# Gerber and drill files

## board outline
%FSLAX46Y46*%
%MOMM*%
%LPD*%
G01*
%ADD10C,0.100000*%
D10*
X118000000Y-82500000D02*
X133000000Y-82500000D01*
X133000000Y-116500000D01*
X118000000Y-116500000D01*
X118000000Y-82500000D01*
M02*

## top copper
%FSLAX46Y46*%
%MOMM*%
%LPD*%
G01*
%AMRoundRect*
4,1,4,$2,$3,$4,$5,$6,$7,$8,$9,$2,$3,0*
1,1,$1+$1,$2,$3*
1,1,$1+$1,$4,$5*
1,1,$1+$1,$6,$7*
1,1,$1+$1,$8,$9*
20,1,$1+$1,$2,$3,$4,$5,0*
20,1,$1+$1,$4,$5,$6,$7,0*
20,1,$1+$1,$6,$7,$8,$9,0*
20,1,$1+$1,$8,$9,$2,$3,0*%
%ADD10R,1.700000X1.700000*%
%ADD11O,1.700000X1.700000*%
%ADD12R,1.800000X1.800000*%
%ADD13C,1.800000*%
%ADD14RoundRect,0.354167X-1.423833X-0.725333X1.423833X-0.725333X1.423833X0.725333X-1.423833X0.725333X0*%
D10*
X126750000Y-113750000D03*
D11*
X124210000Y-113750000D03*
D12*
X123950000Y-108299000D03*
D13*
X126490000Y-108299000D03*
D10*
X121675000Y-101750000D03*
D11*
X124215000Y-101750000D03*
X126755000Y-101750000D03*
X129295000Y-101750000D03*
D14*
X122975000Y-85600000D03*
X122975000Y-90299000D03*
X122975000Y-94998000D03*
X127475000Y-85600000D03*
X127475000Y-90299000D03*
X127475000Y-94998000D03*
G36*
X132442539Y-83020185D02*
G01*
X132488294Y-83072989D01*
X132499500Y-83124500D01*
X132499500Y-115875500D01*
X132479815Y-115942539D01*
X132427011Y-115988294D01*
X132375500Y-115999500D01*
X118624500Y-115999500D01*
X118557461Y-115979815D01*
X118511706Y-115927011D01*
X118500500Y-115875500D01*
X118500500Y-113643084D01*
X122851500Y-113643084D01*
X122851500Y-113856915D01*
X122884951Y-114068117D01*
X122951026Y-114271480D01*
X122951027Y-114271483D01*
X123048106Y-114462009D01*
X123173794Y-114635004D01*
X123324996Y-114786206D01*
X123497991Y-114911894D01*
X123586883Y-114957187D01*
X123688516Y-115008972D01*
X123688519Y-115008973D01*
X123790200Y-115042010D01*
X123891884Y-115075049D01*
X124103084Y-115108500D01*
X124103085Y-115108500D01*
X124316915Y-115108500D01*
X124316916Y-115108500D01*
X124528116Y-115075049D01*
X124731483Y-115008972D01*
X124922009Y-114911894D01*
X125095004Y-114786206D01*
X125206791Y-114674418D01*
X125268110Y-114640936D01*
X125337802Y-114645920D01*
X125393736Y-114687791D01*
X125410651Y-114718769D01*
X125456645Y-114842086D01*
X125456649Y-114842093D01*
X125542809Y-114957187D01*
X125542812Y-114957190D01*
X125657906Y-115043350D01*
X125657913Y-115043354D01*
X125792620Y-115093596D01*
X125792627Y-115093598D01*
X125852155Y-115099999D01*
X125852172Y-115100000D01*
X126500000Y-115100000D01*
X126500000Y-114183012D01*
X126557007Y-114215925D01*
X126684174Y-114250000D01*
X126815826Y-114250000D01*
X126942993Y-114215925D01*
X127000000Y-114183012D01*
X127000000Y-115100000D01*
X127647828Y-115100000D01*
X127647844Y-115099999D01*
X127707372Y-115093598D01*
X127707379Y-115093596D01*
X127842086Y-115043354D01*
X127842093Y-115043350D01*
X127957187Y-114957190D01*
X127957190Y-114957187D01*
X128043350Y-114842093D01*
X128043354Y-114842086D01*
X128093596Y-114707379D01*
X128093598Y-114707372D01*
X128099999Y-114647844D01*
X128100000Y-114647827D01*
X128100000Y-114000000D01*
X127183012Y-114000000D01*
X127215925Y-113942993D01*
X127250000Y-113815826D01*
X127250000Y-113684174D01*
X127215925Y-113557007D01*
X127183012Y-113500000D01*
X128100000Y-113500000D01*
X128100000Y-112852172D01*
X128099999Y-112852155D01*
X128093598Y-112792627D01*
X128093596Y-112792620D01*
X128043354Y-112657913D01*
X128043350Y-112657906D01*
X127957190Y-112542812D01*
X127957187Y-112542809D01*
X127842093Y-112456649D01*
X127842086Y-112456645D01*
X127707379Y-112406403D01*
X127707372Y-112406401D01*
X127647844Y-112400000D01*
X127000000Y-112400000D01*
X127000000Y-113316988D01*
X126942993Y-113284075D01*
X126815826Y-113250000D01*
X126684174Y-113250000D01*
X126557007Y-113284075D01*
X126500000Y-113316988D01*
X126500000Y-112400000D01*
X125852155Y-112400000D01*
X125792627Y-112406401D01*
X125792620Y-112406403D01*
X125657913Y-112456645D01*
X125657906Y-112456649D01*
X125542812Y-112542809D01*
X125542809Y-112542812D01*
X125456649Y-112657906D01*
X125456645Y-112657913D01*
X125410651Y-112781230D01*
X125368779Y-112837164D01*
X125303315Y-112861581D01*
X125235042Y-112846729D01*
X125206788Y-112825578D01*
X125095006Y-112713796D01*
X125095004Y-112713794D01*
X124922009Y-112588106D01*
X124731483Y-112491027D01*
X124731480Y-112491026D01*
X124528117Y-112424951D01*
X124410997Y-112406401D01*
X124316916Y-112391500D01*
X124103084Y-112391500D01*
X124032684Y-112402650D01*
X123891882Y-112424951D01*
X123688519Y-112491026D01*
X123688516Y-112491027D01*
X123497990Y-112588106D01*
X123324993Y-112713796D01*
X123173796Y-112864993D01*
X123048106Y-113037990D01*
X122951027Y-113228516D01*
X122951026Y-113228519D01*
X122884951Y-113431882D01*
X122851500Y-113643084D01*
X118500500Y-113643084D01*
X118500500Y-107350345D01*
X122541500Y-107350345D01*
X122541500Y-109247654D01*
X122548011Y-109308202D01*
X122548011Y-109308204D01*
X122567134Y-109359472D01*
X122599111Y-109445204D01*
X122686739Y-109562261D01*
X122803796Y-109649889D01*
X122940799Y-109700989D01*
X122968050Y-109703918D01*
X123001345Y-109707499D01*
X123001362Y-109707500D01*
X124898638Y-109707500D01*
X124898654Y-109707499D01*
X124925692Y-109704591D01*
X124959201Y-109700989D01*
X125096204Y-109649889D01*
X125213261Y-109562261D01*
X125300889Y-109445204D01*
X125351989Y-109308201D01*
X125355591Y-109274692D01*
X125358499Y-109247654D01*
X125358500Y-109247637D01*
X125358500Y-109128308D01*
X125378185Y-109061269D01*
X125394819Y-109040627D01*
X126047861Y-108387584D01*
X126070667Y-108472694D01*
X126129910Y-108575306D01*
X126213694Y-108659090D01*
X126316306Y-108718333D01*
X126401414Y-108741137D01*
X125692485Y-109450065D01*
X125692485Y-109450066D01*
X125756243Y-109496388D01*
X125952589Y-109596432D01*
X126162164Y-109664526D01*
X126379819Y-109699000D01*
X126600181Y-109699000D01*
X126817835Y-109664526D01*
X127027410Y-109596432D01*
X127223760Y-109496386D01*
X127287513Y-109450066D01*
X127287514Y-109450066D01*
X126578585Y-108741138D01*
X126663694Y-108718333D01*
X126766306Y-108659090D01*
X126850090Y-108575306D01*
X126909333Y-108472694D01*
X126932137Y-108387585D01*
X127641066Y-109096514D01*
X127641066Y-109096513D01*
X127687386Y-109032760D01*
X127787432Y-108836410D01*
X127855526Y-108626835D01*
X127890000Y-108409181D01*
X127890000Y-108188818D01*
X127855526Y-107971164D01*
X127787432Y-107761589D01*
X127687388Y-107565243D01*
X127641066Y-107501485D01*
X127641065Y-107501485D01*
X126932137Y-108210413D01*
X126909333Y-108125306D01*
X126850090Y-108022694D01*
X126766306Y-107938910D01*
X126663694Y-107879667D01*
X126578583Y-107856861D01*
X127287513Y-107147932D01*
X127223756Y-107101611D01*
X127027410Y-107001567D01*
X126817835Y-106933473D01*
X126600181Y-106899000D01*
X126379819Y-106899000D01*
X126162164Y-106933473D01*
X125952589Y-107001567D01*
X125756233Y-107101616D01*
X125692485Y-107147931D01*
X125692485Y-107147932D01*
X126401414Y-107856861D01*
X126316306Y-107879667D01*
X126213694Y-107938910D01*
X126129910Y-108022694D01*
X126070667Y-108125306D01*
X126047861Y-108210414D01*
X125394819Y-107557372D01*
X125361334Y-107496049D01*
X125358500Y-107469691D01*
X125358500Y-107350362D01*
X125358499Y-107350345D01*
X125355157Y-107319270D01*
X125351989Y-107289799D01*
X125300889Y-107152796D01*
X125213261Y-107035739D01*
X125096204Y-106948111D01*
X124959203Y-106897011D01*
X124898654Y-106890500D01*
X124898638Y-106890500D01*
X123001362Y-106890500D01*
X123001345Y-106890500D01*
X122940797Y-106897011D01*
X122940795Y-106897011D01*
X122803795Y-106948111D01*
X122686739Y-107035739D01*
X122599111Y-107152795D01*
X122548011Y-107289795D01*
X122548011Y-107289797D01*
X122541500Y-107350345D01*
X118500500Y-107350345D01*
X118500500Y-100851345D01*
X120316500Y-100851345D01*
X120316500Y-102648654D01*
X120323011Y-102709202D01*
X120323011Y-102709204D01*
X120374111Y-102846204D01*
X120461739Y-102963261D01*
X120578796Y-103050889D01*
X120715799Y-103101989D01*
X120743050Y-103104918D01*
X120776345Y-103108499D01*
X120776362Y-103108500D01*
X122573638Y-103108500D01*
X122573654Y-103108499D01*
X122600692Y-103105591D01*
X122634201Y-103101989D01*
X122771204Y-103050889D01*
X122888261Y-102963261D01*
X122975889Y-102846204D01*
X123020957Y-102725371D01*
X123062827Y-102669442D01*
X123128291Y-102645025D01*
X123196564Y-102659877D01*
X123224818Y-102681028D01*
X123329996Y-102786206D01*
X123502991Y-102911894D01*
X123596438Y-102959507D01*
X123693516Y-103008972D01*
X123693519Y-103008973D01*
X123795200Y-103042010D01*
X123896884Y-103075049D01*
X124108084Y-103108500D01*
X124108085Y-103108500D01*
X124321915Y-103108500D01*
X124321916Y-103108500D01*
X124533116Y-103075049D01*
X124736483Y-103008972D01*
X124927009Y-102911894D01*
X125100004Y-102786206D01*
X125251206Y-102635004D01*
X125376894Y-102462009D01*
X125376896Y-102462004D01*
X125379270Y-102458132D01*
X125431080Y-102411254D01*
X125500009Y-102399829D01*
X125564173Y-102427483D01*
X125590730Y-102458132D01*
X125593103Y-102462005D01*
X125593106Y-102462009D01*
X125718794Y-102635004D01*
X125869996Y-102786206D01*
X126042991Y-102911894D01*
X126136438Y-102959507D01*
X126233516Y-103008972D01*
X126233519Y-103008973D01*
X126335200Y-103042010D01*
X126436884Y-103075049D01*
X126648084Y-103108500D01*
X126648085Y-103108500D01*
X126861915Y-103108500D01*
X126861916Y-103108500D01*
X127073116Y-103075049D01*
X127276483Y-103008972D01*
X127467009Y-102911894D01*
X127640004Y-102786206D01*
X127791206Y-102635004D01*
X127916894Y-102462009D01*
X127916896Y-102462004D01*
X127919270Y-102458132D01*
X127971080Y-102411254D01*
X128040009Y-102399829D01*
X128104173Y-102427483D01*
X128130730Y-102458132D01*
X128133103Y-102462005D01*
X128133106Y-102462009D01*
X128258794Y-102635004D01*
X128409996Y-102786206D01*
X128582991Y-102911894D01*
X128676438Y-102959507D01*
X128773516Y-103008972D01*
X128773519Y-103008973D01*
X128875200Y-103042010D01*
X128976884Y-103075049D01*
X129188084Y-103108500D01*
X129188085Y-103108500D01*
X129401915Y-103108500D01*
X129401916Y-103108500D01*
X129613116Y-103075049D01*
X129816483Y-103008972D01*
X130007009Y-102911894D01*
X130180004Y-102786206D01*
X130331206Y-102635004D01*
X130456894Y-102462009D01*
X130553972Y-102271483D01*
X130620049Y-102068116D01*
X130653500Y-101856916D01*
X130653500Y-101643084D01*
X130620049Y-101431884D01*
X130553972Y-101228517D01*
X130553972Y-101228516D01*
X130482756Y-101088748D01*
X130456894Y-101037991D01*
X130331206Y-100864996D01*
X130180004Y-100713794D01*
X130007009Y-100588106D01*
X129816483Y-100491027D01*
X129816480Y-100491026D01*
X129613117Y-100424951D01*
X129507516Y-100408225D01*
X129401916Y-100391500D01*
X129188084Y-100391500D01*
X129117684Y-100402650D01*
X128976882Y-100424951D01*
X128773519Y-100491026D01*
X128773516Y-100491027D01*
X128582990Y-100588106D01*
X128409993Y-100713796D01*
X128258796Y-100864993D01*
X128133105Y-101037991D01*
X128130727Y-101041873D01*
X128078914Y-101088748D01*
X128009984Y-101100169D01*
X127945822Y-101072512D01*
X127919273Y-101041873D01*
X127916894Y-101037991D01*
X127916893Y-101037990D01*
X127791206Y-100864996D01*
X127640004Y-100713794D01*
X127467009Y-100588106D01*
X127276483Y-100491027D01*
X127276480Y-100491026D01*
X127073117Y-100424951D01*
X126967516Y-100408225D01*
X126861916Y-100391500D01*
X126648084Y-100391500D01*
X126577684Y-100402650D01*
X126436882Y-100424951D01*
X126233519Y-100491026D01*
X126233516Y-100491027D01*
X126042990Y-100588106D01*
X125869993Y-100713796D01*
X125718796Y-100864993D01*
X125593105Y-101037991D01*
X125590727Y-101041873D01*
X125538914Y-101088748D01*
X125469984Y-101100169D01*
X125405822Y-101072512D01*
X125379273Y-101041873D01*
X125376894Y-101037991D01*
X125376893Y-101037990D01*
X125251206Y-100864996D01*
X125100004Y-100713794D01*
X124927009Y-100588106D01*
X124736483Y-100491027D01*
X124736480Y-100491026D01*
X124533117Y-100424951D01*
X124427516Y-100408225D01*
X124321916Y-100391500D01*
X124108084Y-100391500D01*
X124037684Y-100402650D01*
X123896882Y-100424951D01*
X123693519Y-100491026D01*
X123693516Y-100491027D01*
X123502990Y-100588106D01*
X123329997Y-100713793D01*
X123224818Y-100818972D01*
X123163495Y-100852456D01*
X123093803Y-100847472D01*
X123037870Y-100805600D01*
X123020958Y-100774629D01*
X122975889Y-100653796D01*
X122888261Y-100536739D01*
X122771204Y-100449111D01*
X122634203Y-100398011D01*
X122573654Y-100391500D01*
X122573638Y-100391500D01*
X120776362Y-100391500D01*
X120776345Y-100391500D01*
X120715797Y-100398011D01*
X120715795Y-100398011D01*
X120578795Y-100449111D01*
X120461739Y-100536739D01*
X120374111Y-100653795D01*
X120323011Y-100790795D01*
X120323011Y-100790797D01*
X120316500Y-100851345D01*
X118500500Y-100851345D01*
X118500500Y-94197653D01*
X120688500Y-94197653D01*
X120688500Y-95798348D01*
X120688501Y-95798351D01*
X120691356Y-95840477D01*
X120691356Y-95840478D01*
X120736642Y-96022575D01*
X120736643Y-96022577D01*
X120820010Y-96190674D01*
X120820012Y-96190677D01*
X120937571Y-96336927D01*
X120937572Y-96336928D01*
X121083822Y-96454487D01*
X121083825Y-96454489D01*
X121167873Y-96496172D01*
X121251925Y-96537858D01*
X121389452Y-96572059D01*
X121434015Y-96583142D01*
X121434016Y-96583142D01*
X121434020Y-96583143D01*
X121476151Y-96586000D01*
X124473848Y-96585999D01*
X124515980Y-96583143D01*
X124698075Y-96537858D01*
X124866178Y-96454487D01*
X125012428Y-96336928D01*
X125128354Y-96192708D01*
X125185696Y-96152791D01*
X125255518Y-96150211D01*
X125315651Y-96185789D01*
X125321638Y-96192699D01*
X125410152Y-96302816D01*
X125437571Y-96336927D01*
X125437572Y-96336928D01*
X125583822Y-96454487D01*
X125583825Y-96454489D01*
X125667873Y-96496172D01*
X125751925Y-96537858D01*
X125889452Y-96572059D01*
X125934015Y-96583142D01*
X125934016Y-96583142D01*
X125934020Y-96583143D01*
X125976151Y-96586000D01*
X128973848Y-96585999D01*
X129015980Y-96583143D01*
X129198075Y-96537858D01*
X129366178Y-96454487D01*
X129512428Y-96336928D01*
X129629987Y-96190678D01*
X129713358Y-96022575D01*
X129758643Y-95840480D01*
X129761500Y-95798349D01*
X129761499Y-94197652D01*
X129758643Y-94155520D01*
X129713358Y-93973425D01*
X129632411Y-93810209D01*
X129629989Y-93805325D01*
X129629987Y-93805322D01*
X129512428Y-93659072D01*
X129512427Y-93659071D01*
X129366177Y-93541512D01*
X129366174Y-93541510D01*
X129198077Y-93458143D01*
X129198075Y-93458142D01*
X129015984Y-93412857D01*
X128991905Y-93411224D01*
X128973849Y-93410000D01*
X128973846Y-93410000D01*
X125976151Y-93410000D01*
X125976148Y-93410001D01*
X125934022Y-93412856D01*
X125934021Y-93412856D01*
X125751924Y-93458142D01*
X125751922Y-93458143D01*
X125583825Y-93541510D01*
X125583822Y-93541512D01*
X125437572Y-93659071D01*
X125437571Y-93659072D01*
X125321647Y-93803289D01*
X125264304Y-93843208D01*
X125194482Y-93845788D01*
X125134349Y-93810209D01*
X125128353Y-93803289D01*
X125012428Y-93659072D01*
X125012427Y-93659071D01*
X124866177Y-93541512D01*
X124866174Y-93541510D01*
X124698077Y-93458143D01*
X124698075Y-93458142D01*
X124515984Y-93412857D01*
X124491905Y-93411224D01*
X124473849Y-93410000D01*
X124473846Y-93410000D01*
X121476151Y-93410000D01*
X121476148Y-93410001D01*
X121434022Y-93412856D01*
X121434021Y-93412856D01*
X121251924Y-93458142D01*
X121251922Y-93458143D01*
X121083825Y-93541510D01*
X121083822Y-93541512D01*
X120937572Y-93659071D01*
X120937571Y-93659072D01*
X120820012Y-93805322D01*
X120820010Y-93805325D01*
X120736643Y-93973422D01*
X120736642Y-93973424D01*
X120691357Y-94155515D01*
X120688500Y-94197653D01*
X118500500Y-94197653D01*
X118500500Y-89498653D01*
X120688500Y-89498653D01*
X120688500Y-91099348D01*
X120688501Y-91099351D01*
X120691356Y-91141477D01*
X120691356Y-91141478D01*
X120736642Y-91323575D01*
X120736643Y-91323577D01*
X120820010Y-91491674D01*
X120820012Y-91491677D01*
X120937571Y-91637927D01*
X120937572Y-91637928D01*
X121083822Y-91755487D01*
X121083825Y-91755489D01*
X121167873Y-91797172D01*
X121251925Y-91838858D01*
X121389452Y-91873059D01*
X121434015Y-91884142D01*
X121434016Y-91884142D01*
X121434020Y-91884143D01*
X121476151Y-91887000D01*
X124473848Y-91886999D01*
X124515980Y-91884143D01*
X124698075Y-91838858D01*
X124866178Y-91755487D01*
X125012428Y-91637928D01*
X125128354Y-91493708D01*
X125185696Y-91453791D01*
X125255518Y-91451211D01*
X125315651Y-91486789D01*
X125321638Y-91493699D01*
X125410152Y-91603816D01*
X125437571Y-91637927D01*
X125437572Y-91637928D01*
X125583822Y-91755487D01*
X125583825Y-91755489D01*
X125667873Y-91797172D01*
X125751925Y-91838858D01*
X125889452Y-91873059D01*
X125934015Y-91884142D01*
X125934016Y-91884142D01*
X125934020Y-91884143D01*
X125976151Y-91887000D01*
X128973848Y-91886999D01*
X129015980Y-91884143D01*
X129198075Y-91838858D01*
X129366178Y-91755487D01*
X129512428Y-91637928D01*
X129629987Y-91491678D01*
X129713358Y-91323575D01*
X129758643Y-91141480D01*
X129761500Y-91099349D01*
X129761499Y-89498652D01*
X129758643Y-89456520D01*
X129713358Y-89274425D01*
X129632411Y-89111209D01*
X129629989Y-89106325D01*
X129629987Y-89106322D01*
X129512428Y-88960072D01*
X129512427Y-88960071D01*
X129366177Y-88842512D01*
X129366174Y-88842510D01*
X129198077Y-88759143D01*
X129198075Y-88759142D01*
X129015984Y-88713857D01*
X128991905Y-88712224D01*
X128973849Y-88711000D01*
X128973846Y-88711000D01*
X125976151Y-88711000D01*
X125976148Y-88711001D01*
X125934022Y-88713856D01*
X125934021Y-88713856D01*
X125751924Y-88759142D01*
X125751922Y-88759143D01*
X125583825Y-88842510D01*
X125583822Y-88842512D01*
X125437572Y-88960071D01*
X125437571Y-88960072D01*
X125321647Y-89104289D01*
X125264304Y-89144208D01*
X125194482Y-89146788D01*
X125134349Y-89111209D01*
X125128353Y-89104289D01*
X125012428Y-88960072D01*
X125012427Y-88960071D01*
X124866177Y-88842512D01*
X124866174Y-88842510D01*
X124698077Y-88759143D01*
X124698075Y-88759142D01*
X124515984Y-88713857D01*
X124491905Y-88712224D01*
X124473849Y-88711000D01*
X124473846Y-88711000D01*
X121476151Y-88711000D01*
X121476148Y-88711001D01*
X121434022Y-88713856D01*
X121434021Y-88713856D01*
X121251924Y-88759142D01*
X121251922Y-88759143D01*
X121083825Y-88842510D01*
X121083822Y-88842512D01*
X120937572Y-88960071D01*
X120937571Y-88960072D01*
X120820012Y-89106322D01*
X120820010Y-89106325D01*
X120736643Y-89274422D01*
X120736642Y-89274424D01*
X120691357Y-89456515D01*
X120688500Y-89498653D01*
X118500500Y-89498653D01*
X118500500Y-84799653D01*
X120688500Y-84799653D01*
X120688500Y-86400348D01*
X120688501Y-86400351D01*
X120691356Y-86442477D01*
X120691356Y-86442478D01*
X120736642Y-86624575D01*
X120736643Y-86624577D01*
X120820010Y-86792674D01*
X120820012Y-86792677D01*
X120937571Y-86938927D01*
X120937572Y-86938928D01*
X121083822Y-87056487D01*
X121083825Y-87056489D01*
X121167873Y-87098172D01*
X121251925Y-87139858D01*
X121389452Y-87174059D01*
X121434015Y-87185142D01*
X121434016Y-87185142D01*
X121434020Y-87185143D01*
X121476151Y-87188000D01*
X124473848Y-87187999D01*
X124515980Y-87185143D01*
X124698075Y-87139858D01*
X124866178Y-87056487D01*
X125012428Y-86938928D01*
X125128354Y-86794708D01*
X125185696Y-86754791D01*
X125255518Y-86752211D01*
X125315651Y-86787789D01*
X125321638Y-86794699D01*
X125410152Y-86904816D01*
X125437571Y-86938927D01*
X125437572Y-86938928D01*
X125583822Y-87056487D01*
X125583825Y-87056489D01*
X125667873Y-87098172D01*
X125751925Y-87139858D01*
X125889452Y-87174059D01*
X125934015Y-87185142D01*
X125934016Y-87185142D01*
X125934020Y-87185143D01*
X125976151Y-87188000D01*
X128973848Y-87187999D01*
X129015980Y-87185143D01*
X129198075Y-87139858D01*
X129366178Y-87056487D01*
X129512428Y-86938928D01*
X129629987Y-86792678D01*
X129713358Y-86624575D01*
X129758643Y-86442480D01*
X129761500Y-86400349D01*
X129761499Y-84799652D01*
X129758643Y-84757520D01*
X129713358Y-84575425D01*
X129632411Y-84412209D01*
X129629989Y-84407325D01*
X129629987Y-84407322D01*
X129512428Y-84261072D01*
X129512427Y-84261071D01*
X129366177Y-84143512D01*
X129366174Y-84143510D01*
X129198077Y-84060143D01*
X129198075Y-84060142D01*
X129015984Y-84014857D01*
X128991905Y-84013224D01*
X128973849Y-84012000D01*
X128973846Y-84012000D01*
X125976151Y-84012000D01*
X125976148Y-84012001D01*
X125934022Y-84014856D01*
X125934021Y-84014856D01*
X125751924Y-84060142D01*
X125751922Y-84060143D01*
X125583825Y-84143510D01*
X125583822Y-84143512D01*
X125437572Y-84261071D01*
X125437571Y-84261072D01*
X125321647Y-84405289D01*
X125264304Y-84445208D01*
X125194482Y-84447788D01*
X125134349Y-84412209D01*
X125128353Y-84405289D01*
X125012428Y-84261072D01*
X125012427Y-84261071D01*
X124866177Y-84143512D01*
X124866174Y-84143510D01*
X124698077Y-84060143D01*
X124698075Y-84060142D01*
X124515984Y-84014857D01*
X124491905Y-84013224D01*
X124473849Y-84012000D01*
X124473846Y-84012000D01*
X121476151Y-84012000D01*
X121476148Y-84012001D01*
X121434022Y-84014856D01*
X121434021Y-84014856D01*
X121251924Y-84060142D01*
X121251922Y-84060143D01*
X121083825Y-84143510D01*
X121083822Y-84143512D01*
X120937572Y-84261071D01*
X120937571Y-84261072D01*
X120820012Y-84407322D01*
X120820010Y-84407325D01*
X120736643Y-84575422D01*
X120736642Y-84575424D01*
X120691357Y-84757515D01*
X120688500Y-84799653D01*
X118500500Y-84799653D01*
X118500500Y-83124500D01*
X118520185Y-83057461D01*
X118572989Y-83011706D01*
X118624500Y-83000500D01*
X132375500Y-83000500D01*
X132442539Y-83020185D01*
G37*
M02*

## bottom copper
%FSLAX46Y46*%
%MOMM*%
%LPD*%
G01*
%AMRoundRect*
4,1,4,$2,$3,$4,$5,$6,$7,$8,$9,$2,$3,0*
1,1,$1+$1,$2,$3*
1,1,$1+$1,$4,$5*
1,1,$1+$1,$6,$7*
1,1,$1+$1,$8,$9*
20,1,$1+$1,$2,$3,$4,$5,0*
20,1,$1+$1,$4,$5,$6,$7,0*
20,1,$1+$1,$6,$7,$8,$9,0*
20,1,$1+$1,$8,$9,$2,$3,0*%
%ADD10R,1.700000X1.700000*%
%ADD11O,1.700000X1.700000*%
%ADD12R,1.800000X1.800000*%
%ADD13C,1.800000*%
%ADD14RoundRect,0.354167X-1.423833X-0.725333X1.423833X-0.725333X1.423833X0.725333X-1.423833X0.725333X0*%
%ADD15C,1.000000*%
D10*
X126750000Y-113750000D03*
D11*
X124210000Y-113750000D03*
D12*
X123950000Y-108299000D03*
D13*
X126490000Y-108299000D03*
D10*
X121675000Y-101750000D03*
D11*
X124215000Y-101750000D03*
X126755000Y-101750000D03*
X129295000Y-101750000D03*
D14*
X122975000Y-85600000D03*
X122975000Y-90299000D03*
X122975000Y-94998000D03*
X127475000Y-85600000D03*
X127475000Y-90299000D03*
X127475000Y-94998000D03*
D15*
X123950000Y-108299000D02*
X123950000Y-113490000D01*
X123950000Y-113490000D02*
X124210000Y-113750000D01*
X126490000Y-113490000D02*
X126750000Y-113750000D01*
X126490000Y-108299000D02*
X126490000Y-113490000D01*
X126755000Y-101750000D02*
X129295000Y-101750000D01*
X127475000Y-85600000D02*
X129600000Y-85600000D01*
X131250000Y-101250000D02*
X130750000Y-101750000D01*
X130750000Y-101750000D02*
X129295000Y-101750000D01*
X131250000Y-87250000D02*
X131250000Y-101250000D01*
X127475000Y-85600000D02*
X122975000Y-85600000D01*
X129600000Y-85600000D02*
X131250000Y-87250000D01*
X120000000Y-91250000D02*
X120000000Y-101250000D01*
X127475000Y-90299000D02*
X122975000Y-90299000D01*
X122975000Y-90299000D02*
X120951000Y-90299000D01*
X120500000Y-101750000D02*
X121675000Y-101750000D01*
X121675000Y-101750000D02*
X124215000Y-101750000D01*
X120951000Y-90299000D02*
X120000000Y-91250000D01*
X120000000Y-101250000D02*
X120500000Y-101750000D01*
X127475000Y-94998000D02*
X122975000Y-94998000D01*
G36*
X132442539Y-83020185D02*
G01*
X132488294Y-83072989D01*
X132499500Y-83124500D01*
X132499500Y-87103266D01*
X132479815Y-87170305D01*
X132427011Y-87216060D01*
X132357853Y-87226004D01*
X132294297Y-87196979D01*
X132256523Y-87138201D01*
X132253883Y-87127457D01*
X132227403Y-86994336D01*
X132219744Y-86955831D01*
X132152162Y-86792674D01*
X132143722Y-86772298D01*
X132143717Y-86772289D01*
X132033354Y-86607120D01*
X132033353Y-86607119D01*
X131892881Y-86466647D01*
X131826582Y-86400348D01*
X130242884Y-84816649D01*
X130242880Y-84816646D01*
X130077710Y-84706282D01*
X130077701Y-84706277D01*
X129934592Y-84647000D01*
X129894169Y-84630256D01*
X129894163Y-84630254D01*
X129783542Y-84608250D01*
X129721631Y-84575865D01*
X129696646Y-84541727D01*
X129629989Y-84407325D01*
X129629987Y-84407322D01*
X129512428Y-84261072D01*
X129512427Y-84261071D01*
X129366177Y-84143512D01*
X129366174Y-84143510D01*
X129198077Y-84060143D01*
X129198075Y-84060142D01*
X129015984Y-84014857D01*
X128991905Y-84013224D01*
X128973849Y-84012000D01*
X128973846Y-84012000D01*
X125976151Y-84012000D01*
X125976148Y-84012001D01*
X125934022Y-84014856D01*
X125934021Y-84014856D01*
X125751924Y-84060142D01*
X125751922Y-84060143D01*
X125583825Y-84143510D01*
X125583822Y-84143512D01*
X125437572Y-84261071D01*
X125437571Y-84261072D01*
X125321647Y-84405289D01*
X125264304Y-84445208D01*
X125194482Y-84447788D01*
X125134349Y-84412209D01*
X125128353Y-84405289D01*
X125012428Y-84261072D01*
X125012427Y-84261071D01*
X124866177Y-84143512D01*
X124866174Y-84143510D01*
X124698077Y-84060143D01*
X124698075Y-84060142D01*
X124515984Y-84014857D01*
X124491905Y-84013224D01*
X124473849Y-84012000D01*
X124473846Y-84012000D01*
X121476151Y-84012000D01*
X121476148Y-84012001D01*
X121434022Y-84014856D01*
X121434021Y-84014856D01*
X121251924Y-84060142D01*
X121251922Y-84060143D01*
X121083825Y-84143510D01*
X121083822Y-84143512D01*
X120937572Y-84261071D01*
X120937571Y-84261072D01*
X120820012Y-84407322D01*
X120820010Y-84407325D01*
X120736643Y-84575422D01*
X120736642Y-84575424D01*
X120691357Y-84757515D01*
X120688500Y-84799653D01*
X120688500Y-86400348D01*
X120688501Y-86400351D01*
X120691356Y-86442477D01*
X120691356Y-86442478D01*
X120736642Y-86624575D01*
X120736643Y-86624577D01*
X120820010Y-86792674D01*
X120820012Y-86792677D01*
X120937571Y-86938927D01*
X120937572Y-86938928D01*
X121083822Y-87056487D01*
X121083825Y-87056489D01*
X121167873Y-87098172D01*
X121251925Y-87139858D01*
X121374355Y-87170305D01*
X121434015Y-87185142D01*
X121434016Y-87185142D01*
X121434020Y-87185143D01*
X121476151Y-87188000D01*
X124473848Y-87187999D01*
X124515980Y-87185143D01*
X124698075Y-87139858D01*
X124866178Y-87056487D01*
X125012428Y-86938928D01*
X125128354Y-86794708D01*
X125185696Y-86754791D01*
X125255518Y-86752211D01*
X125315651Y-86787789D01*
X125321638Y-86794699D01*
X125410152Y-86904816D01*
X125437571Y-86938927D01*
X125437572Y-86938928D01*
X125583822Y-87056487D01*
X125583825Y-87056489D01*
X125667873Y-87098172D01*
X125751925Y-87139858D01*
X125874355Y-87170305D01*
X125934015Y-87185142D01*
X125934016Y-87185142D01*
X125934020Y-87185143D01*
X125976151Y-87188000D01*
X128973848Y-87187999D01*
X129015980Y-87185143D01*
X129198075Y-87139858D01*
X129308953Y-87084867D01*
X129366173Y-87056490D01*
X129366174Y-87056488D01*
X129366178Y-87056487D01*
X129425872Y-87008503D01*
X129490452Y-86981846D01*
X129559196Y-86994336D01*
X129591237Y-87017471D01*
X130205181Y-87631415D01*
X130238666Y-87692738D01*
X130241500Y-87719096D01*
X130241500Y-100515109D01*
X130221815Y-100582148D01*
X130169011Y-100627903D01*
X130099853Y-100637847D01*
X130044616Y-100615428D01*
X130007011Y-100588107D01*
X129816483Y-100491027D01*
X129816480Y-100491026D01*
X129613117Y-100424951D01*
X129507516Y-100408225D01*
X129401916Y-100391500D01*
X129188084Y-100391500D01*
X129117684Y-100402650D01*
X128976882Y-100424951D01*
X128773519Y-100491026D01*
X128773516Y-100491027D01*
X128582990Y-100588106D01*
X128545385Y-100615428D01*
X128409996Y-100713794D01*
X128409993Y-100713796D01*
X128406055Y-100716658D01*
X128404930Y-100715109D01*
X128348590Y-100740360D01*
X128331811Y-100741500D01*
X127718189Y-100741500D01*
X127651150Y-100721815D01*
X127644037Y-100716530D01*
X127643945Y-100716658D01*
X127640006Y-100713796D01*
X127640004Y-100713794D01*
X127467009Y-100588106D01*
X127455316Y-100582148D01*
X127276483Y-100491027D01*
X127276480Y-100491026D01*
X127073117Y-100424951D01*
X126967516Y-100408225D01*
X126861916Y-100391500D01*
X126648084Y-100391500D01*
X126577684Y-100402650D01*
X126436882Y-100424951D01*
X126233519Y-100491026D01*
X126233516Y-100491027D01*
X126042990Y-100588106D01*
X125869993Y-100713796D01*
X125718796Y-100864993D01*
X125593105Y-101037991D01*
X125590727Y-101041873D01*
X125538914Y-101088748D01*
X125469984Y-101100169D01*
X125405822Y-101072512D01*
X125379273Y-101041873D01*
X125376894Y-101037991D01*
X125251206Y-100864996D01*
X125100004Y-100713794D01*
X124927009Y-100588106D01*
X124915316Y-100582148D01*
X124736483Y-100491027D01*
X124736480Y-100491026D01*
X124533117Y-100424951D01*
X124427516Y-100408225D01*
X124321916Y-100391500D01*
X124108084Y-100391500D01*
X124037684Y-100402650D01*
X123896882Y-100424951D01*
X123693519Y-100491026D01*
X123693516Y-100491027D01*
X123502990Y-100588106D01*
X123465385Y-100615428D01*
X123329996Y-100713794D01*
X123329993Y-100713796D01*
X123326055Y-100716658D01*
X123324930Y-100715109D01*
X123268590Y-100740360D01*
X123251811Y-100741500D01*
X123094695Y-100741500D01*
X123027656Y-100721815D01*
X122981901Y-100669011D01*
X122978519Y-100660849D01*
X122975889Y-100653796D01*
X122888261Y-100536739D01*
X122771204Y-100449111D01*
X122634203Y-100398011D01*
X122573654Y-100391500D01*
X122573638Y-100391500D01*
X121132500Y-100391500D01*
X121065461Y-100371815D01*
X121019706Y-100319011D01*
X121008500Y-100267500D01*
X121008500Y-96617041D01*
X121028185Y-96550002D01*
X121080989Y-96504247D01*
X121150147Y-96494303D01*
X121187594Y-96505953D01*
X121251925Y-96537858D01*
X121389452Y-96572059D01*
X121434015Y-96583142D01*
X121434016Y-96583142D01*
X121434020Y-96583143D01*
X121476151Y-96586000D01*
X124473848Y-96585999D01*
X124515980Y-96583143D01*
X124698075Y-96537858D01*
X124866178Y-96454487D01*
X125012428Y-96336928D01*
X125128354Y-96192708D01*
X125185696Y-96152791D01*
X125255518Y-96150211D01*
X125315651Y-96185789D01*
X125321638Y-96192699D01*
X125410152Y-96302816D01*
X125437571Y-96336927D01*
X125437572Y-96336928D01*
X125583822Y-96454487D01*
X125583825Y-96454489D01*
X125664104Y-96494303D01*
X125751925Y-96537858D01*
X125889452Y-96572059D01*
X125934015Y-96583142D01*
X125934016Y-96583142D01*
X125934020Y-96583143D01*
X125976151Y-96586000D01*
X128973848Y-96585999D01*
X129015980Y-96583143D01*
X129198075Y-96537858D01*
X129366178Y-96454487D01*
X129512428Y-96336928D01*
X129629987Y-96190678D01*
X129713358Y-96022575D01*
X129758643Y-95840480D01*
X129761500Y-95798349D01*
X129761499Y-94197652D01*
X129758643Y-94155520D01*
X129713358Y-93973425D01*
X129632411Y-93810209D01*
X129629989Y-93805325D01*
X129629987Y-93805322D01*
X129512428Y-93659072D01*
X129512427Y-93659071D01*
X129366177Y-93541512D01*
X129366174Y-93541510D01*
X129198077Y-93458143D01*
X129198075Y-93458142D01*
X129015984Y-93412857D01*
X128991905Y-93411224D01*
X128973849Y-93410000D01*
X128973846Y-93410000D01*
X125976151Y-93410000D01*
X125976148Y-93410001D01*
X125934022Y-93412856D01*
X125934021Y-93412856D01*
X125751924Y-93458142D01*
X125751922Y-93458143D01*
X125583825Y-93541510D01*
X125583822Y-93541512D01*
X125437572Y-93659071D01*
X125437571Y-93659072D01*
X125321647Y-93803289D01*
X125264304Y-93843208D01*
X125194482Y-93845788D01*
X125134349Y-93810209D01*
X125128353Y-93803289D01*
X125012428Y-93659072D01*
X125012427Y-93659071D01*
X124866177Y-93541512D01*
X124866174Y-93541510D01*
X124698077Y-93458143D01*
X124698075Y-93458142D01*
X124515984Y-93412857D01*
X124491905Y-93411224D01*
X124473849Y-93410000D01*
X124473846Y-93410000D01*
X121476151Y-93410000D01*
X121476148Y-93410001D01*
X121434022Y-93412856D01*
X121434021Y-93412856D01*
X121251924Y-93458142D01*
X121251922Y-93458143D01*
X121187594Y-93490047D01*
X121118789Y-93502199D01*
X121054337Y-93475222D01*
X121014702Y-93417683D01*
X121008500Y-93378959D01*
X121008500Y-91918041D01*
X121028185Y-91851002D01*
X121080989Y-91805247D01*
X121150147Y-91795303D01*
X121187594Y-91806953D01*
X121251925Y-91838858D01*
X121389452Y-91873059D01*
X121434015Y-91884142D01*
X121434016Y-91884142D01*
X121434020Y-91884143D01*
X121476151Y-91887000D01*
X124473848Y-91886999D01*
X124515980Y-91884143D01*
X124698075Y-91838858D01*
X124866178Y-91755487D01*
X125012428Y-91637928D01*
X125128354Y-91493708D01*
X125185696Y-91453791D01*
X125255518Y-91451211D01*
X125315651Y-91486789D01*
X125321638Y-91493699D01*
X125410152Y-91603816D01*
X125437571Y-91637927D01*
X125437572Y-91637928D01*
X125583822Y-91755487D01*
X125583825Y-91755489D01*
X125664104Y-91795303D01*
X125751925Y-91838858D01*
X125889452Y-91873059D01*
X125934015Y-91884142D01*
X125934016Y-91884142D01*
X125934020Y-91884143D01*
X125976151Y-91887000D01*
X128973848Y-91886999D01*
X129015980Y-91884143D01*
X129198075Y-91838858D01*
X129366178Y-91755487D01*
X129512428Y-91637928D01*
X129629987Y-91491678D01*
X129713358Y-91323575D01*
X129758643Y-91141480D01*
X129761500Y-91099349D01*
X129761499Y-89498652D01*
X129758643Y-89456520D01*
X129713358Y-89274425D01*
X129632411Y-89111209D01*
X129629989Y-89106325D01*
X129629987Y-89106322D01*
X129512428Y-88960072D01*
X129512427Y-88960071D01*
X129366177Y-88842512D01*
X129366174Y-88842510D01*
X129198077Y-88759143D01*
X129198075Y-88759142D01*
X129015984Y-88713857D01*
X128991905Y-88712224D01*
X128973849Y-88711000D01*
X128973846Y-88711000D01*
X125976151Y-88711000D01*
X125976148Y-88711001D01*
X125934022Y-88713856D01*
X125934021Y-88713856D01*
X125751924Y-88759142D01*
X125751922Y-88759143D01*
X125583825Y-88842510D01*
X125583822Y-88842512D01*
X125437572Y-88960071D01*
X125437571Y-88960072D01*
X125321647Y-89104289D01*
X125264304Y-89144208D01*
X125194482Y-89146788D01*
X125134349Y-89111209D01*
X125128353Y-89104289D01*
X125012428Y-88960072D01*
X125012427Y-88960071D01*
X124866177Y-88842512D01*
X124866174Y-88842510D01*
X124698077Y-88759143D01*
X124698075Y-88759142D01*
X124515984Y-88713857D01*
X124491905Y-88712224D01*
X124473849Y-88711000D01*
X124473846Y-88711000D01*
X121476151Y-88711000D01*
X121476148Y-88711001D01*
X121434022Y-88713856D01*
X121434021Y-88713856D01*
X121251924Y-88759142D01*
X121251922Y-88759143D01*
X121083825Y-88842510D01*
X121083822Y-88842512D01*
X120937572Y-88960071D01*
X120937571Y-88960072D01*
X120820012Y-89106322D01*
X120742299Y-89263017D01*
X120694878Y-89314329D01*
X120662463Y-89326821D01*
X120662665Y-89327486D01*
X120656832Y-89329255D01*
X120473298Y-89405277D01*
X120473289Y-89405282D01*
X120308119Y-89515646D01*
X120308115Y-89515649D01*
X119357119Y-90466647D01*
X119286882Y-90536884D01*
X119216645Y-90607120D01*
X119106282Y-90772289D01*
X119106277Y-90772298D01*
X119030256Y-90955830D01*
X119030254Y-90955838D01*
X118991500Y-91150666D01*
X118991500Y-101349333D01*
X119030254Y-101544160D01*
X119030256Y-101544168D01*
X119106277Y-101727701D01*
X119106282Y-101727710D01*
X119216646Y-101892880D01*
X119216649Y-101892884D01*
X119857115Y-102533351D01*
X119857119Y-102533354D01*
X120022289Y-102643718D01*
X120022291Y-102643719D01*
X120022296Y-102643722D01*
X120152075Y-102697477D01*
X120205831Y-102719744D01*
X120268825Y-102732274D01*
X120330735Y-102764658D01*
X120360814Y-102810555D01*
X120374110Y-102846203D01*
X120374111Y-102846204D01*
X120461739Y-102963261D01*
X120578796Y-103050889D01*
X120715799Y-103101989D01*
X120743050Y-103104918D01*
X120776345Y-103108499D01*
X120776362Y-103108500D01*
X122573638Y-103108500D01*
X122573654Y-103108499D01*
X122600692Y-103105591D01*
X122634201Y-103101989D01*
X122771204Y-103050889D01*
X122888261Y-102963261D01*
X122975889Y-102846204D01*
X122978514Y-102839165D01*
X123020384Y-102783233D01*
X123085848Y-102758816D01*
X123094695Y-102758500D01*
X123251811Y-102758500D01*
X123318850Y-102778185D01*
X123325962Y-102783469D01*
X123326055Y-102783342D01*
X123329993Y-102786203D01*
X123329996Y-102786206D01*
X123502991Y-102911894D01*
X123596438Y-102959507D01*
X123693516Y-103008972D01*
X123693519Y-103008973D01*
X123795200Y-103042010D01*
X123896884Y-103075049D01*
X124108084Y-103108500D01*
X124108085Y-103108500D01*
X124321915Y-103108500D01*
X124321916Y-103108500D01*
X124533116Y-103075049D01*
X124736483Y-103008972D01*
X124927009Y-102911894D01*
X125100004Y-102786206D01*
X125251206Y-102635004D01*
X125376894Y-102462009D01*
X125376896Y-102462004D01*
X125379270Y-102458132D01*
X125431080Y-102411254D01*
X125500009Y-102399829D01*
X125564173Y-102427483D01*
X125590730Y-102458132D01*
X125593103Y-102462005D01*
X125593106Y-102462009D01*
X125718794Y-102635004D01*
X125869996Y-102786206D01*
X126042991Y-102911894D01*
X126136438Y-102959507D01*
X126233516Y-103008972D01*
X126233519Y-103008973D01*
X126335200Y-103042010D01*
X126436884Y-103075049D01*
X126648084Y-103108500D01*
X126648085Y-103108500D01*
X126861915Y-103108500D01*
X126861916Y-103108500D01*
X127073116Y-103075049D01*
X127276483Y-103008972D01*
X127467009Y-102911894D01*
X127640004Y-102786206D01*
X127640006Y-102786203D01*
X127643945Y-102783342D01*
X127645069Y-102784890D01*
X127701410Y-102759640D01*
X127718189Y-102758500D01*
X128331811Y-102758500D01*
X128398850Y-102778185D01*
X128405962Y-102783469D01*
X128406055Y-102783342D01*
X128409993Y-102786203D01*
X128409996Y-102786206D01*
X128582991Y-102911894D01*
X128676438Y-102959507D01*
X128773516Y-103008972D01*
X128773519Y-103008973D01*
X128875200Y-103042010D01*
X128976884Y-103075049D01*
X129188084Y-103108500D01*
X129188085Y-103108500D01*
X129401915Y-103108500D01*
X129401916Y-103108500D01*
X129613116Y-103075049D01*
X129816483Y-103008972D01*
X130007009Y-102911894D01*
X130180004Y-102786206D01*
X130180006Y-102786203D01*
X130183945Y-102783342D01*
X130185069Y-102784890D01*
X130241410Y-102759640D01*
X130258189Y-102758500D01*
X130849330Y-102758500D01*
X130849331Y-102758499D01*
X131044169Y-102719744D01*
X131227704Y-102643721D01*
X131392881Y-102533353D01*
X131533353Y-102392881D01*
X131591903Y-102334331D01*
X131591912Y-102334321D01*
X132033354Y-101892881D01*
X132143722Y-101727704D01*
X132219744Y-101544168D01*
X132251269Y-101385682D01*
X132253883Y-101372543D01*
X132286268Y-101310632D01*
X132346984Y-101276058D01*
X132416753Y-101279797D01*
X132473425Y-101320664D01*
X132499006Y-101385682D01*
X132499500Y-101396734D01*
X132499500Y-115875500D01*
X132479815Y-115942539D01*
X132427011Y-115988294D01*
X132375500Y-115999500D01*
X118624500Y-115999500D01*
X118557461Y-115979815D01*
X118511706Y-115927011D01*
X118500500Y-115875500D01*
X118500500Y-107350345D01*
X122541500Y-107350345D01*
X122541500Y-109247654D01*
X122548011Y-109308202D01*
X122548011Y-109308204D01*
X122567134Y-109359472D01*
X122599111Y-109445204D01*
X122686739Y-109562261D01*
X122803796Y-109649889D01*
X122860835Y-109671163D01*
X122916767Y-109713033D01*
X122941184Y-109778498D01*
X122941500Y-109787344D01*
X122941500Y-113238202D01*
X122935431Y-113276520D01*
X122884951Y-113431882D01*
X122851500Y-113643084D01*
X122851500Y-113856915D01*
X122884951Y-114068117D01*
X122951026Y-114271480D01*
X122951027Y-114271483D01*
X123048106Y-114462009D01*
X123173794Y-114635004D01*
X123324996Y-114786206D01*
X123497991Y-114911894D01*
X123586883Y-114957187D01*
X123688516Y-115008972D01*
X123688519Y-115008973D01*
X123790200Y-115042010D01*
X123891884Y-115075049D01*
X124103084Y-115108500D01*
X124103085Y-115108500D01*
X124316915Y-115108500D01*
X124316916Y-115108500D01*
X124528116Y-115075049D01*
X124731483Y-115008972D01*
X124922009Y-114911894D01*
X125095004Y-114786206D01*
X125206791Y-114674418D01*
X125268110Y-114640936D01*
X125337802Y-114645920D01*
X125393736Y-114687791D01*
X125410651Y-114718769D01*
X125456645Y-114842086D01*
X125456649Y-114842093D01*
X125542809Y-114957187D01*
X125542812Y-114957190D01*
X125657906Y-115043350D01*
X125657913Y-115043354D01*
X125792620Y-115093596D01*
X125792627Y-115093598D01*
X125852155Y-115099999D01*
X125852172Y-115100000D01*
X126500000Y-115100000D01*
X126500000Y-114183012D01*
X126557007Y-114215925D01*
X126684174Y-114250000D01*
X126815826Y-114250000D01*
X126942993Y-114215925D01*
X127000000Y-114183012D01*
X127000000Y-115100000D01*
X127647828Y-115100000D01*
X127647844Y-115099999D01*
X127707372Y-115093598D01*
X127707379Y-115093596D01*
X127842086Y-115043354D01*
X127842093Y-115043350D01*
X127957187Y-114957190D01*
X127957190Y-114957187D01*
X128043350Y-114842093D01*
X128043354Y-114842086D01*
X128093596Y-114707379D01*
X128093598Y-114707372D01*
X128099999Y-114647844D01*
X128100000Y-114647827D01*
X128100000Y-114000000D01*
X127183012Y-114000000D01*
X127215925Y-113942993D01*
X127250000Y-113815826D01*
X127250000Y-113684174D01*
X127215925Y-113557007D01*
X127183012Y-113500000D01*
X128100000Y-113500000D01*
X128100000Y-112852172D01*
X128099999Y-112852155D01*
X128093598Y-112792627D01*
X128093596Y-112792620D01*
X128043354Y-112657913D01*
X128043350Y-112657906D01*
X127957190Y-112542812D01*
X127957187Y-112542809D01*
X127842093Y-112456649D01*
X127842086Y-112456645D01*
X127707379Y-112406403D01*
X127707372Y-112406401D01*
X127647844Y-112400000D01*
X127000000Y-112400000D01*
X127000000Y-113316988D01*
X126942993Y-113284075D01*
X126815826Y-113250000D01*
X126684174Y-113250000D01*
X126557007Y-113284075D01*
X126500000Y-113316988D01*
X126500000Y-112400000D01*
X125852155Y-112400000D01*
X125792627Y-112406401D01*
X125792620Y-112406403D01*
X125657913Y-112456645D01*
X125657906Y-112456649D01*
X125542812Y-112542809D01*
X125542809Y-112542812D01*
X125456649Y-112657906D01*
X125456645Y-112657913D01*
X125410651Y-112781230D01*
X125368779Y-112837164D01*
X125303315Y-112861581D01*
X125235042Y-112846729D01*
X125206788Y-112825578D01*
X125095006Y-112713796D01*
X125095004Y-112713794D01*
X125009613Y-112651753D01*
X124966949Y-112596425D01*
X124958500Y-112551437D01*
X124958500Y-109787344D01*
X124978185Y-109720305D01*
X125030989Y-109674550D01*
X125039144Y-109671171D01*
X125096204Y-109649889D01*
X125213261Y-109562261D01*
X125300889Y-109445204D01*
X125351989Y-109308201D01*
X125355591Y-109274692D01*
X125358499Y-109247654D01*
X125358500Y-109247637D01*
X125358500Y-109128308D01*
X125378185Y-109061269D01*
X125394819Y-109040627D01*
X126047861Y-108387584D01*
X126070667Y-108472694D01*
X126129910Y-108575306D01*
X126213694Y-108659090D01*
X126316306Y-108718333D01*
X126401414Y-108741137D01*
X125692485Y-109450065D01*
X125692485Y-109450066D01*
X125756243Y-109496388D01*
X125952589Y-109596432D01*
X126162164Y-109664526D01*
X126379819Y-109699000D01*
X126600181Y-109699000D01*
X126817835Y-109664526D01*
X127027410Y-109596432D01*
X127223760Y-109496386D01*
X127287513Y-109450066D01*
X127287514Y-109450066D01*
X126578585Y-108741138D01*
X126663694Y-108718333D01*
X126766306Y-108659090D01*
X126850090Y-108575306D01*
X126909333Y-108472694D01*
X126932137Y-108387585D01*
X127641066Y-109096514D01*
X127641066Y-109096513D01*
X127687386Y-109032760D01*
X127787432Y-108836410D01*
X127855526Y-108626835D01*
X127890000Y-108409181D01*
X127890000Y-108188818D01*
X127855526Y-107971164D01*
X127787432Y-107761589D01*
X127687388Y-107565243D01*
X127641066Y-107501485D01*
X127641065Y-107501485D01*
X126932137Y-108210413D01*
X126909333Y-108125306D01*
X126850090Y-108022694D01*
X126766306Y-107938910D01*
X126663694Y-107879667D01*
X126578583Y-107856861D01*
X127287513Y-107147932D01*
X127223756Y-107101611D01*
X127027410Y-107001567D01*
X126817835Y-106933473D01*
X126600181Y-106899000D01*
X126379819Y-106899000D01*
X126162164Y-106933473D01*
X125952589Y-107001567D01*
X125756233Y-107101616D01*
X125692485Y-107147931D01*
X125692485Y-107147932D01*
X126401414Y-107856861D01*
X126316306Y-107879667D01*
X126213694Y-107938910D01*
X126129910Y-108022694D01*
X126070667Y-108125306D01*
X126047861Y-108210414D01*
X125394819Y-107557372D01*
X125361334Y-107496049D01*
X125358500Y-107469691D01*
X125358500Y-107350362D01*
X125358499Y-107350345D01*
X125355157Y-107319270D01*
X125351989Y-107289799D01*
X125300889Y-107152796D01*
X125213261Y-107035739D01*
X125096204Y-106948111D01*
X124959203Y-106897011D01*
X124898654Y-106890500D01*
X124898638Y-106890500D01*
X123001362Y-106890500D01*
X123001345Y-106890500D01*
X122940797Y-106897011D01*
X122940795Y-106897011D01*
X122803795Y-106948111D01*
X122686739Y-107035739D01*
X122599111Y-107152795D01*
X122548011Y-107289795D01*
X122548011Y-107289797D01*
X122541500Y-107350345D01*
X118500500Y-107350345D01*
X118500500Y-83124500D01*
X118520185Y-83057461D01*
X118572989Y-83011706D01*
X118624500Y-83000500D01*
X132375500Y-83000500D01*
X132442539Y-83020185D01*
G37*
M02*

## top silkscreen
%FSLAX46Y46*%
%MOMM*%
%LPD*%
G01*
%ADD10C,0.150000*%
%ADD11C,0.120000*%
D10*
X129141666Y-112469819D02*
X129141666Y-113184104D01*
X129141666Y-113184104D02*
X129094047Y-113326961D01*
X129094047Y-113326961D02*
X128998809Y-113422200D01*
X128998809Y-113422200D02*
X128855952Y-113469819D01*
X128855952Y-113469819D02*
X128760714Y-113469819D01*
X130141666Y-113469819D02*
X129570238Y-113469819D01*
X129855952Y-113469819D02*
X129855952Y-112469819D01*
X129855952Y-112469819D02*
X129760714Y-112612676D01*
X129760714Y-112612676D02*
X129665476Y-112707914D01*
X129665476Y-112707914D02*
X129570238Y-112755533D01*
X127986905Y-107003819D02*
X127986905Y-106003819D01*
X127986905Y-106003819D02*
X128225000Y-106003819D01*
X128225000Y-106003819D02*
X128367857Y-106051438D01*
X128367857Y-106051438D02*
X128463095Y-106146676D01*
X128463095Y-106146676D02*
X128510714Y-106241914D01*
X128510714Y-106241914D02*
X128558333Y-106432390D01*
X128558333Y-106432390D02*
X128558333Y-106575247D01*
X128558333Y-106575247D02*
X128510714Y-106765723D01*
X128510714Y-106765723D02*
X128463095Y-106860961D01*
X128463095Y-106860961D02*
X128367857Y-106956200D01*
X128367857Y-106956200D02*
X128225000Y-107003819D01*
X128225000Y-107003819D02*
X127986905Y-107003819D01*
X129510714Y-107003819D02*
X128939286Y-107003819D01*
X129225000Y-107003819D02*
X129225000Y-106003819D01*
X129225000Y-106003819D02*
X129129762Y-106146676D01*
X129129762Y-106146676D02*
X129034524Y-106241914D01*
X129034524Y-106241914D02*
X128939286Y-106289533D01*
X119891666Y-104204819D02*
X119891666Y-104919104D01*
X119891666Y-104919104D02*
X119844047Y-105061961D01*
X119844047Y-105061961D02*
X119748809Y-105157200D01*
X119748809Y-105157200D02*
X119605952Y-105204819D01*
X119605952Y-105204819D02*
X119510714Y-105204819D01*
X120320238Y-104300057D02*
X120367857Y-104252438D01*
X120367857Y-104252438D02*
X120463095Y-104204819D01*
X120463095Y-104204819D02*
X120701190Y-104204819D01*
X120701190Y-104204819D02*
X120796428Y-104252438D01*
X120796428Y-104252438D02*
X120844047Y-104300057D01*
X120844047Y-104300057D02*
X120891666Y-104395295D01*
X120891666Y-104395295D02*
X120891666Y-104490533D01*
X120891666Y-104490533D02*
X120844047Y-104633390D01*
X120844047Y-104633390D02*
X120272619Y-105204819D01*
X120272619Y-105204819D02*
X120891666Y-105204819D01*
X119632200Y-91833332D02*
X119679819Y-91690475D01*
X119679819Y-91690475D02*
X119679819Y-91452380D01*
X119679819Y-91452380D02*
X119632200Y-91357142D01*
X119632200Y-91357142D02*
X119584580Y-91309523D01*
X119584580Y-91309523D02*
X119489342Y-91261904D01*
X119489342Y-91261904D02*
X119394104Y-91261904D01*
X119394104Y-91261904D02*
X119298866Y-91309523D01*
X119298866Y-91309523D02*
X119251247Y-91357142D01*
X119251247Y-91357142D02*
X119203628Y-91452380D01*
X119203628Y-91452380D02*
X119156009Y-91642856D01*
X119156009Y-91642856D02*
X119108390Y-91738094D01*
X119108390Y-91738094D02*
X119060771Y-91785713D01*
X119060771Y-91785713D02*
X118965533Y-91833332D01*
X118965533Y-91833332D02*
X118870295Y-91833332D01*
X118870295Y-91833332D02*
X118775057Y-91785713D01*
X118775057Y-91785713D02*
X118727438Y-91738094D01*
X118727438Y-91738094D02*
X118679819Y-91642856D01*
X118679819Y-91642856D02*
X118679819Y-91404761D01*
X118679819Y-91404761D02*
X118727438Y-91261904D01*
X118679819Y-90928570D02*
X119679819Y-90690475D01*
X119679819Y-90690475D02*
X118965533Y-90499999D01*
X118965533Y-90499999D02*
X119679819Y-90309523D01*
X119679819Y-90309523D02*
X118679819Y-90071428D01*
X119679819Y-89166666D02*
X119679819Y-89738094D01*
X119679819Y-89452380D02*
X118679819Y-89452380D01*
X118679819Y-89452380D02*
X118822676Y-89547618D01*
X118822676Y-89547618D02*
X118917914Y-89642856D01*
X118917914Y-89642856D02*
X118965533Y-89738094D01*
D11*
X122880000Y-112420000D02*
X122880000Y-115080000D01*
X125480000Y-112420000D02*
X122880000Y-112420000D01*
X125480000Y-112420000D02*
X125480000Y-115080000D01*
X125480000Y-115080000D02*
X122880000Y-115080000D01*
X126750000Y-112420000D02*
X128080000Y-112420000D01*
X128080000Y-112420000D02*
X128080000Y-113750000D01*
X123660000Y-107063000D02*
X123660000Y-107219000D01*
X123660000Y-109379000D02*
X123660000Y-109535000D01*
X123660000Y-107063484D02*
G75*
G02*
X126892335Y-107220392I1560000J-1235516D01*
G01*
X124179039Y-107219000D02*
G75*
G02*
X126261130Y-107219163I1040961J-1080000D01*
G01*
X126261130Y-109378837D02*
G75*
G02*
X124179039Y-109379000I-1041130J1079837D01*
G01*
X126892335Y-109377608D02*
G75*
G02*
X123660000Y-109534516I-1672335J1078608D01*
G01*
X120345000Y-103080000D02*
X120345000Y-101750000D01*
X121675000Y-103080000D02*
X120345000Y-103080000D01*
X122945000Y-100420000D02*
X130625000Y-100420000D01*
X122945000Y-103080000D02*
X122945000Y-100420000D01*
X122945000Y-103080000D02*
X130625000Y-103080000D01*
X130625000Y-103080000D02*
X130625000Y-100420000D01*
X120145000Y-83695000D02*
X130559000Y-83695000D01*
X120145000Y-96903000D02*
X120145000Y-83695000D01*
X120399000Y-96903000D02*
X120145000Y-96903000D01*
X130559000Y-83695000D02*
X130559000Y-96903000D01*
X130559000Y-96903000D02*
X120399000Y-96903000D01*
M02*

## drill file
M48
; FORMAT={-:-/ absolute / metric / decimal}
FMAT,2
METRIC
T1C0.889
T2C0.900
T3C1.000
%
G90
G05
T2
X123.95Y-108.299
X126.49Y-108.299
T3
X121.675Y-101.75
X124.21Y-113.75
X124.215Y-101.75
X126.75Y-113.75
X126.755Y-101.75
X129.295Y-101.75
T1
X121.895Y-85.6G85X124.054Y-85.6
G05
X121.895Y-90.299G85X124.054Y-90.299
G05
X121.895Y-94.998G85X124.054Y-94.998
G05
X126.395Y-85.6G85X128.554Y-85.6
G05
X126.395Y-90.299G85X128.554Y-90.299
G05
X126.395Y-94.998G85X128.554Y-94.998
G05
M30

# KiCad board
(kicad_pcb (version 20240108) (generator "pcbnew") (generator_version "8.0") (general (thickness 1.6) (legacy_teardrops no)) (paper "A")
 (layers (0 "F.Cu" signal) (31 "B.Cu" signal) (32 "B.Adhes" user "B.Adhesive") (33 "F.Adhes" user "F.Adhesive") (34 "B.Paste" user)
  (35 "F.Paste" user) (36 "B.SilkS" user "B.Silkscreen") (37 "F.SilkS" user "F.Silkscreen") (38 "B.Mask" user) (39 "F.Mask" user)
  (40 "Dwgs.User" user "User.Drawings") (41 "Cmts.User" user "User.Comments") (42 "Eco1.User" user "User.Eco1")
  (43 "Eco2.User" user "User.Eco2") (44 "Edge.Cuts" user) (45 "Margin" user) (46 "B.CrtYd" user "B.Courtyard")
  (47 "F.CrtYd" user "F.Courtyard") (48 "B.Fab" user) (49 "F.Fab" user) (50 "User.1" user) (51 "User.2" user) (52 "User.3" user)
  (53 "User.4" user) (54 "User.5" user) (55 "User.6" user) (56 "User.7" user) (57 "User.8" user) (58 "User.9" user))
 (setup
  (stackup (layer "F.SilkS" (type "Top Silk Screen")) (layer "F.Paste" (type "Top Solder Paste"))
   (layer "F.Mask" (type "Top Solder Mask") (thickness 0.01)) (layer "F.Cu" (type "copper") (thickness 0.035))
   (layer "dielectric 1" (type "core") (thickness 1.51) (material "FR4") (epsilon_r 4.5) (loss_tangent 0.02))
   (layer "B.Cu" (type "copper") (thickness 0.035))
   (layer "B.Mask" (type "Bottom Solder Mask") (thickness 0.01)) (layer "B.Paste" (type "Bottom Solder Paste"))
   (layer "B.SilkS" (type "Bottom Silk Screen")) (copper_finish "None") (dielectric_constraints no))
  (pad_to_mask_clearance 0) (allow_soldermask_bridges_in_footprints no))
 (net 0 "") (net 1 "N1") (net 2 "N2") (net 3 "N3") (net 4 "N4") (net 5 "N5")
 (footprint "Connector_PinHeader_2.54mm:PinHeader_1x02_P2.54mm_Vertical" (layer "F.Cu") (at 126.75 113.75 -90)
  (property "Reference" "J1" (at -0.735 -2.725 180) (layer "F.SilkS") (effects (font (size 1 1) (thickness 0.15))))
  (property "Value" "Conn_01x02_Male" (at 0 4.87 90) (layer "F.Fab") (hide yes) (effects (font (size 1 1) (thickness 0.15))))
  (fp_line (start -1.33 3.87) (end 1.33 3.87) (stroke (width 0.12) (type solid)) (layer "F.SilkS"))
  (fp_line (start -1.33 1.27) (end -1.33 3.87) (stroke (width 0.12) (type solid)) (layer "F.SilkS"))
  (fp_line (start -1.33 1.27) (end 1.33 1.27) (stroke (width 0.12) (type solid)) (layer "F.SilkS"))
  (fp_line (start 1.33 1.27) (end 1.33 3.87) (stroke (width 0.12) (type solid)) (layer "F.SilkS"))
  (fp_line (start -1.33 0) (end -1.33 -1.33) (stroke (width 0.12) (type solid)) (layer "F.SilkS"))
  (fp_line (start -1.33 -1.33) (end 0 -1.33) (stroke (width 0.12) (type solid)) (layer "F.SilkS"))
  (pad "1" thru_hole rect (at 0 0 270) (size 1.7 1.7) (drill 1) (layers "*.Cu" "*.Mask") (remove_unused_layers no) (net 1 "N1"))
  (pad "2" thru_hole oval (at 0 2.54 270) (size 1.7 1.7) (drill 1) (layers "*.Cu" "*.Mask") (remove_unused_layers no) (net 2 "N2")))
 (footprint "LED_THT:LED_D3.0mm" (layer "F.Cu") (at 123.95 108.299)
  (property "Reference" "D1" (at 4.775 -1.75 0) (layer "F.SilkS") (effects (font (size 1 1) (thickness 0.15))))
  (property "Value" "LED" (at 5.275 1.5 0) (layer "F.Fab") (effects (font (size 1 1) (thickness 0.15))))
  (fp_line (start -0.29 -1.236) (end -0.29 -1.08) (stroke (width 0.12) (type solid)) (layer "F.SilkS"))
  (fp_line (start -0.29 1.08) (end -0.29 1.236) (stroke (width 0.12) (type solid)) (layer "F.SilkS"))
  (fp_arc (start -0.29 -1.235516) (mid 1.366487 -1.987659) (end 2.942335 -1.078608) (stroke (width 0.12) (type solid)) (layer "F.SilkS"))
  (fp_arc (start 0.229039 -1.08) (mid 1.270117 -1.5) (end 2.31113 -1.079837) (stroke (width 0.12) (type solid)) (layer "F.SilkS"))
  (fp_arc (start 2.31113 1.079837) (mid 1.270117 1.5) (end 0.229039 1.08) (stroke (width 0.12) (type solid)) (layer "F.SilkS"))
  (fp_arc (start 2.942335 1.078608) (mid 1.366487 1.987659) (end -0.29 1.235516) (stroke (width 0.12) (type solid)) (layer "F.SilkS"))
  (pad "1" thru_hole rect (at 0 0) (size 1.8 1.8) (drill 0.9) (layers "*.Cu" "*.Mask") (remove_unused_layers no) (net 2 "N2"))
  (pad "2" thru_hole circle (at 2.54 0) (size 1.8 1.8) (drill 0.9) (layers "*.Cu" "*.Mask") (remove_unused_layers no) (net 1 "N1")))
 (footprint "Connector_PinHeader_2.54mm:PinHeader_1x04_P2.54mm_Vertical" (layer "F.Cu") (at 121.675 101.75 90)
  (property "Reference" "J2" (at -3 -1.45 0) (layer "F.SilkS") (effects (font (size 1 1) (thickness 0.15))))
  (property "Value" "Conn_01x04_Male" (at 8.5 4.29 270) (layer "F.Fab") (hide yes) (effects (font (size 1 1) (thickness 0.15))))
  (fp_line (start -1.33 -1.33) (end 0 -1.33) (stroke (width 0.12) (type solid)) (layer "F.SilkS"))
  (fp_line (start -1.33 0) (end -1.33 -1.33) (stroke (width 0.12) (type solid)) (layer "F.SilkS"))
  (fp_line (start 1.33 1.27) (end 1.33 8.95) (stroke (width 0.12) (type solid)) (layer "F.SilkS"))
  (fp_line (start -1.33 1.27) (end 1.33 1.27) (stroke (width 0.12) (type solid)) (layer "F.SilkS"))
  (fp_line (start -1.33 1.27) (end -1.33 8.95) (stroke (width 0.12) (type solid)) (layer "F.SilkS"))
  (fp_line (start -1.33 8.95) (end 1.33 8.95) (stroke (width 0.12) (type solid)) (layer "F.SilkS"))
  (pad "1" thru_hole rect (at 0 0 90) (size 1.7 1.7) (drill 1) (layers "*.Cu" "*.Mask") (remove_unused_layers no) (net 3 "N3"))
  (pad "2" thru_hole oval (at 0 2.54 90) (size 1.7 1.7) (drill 1) (layers "*.Cu" "*.Mask") (remove_unused_layers no) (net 3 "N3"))
  (pad "3" thru_hole oval (at 0 5.08 90) (size 1.7 1.7) (drill 1) (layers "*.Cu" "*.Mask") (remove_unused_layers no) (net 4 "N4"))
  (pad "4" thru_hole oval (at 0 7.62 90) (size 1.7 1.7) (drill 1) (layers "*.Cu" "*.Mask") (remove_unused_layers no) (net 4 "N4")))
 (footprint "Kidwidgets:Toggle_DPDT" (layer "F.Cu") (at 125.225 90.299)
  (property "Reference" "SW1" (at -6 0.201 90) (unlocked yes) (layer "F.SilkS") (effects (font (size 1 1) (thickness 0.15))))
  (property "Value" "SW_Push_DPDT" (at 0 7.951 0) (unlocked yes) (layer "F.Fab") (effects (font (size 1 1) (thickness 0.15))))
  (fp_line (start -5.08 -6.604) (end 5.334 -6.604) (stroke (width 0.12) (type default)) (layer "F.SilkS"))
  (fp_line (start -5.08 6.604) (end -5.08 -6.604) (stroke (width 0.12) (type default)) (layer "F.SilkS"))
  (fp_line (start -4.826 6.604) (end -5.08 6.604) (stroke (width 0.12) (type default)) (layer "F.SilkS"))
  (fp_line (start 5.334 -6.604) (end 5.334 6.604) (stroke (width 0.12) (type default)) (layer "F.SilkS"))
  (fp_line (start 5.334 6.604) (end -4.826 6.604) (stroke (width 0.12) (type default)) (layer "F.SilkS"))
  (pad "1" thru_hole roundrect (at -2.25 -4.699) (size 3.556 2.159) (drill oval 3.048 0.889) (layers "*.Cu" "*.Mask")
   (remove_unused_layers no) (roundrect_rratio 0.1640421491) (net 4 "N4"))
  (pad "2" thru_hole roundrect (at -2.25 0) (size 3.556 2.159) (drill oval 3.048 0.889) (layers "*.Cu" "*.Mask") (remove_unused_layers no)
   (roundrect_rratio 0.1640421491) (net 3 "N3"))
  (pad "3" thru_hole roundrect (at -2.25 4.699) (size 3.556 2.159) (drill oval 3.048 0.889) (layers "*.Cu" "*.Mask")
   (remove_unused_layers no) (roundrect_rratio 0.1640421491) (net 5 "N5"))
  (pad "4" thru_hole roundrect (at 2.25 -4.699) (size 3.556 2.159) (drill oval 3.048 0.889) (layers "*.Cu" "*.Mask")
   (remove_unused_layers no) (roundrect_rratio 0.1640421491) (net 4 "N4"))
  (pad "5" thru_hole roundrect (at 2.25 0) (size 3.556 2.159) (drill oval 3.048 0.889) (layers "*.Cu" "*.Mask") (remove_unused_layers no)
   (roundrect_rratio 0.1640421491) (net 3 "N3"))
  (pad "6" thru_hole roundrect (at 2.25 4.699) (size 3.556 2.159) (drill oval 3.048 0.889) (layers "*.Cu" "*.Mask")
   (remove_unused_layers no) (roundrect_rratio 0.1640421491) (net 5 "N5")))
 (gr_rect (start 118 82.5) (end 133 116.5) (stroke (width 0.1) (type default)) (fill none) (layer "Edge.Cuts"))
 (segment (start 123.95 108.299) (end 123.95 113.49) (width 1) (layer "B.Cu") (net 2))
 (segment (start 123.95 113.49) (end 124.21 113.75) (width 1) (layer "B.Cu") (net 2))
 (segment (start 126.49 113.49) (end 126.75 113.75) (width 1) (layer "B.Cu") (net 1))
 (segment (start 126.49 108.299) (end 126.49 113.49) (width 1) (layer "B.Cu") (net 1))
 (segment (start 126.755 101.75) (end 129.295 101.75) (width 1) (layer "B.Cu") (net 4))
 (segment (start 127.475 85.6) (end 129.6 85.6) (width 1) (layer "B.Cu") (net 4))
 (segment (start 131.25 101.25) (end 130.75 101.75) (width 1) (layer "B.Cu") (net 4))
 (segment (start 130.75 101.75) (end 129.295 101.75) (width 1) (layer "B.Cu") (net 4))
 (segment (start 131.25 87.25) (end 131.25 101.25) (width 1) (layer "B.Cu") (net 4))
 (segment (start 127.475 85.6) (end 122.975 85.6) (width 1) (layer "B.Cu") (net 4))
 (segment (start 129.6 85.6) (end 131.25 87.25) (width 1) (layer "B.Cu") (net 4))
 (segment (start 120 91.25) (end 120 101.25) (width 1) (layer "B.Cu") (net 3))
 (segment (start 127.475 90.299) (end 122.975 90.299) (width 1) (layer "B.Cu") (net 3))
 (segment (start 122.975 90.299) (end 120.951 90.299) (width 1) (layer "B.Cu") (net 3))
 (segment (start 120.5 101.75) (end 121.675 101.75) (width 1) (layer "B.Cu") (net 3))
 (segment (start 121.675 101.75) (end 124.215 101.75) (width 1) (layer "B.Cu") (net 3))
 (segment (start 120.951 90.299) (end 120 91.25) (width 1) (layer "B.Cu") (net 3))
 (segment (start 120 101.25) (end 120.5 101.75) (width 1) (layer "B.Cu") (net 3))
 (segment (start 127.475 94.998) (end 122.975 94.998) (width 1) (layer "B.Cu") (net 5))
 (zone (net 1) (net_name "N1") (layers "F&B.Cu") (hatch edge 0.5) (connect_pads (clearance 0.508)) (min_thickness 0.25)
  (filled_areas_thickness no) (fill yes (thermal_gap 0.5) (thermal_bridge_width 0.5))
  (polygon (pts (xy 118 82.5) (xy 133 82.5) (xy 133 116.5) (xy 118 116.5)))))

